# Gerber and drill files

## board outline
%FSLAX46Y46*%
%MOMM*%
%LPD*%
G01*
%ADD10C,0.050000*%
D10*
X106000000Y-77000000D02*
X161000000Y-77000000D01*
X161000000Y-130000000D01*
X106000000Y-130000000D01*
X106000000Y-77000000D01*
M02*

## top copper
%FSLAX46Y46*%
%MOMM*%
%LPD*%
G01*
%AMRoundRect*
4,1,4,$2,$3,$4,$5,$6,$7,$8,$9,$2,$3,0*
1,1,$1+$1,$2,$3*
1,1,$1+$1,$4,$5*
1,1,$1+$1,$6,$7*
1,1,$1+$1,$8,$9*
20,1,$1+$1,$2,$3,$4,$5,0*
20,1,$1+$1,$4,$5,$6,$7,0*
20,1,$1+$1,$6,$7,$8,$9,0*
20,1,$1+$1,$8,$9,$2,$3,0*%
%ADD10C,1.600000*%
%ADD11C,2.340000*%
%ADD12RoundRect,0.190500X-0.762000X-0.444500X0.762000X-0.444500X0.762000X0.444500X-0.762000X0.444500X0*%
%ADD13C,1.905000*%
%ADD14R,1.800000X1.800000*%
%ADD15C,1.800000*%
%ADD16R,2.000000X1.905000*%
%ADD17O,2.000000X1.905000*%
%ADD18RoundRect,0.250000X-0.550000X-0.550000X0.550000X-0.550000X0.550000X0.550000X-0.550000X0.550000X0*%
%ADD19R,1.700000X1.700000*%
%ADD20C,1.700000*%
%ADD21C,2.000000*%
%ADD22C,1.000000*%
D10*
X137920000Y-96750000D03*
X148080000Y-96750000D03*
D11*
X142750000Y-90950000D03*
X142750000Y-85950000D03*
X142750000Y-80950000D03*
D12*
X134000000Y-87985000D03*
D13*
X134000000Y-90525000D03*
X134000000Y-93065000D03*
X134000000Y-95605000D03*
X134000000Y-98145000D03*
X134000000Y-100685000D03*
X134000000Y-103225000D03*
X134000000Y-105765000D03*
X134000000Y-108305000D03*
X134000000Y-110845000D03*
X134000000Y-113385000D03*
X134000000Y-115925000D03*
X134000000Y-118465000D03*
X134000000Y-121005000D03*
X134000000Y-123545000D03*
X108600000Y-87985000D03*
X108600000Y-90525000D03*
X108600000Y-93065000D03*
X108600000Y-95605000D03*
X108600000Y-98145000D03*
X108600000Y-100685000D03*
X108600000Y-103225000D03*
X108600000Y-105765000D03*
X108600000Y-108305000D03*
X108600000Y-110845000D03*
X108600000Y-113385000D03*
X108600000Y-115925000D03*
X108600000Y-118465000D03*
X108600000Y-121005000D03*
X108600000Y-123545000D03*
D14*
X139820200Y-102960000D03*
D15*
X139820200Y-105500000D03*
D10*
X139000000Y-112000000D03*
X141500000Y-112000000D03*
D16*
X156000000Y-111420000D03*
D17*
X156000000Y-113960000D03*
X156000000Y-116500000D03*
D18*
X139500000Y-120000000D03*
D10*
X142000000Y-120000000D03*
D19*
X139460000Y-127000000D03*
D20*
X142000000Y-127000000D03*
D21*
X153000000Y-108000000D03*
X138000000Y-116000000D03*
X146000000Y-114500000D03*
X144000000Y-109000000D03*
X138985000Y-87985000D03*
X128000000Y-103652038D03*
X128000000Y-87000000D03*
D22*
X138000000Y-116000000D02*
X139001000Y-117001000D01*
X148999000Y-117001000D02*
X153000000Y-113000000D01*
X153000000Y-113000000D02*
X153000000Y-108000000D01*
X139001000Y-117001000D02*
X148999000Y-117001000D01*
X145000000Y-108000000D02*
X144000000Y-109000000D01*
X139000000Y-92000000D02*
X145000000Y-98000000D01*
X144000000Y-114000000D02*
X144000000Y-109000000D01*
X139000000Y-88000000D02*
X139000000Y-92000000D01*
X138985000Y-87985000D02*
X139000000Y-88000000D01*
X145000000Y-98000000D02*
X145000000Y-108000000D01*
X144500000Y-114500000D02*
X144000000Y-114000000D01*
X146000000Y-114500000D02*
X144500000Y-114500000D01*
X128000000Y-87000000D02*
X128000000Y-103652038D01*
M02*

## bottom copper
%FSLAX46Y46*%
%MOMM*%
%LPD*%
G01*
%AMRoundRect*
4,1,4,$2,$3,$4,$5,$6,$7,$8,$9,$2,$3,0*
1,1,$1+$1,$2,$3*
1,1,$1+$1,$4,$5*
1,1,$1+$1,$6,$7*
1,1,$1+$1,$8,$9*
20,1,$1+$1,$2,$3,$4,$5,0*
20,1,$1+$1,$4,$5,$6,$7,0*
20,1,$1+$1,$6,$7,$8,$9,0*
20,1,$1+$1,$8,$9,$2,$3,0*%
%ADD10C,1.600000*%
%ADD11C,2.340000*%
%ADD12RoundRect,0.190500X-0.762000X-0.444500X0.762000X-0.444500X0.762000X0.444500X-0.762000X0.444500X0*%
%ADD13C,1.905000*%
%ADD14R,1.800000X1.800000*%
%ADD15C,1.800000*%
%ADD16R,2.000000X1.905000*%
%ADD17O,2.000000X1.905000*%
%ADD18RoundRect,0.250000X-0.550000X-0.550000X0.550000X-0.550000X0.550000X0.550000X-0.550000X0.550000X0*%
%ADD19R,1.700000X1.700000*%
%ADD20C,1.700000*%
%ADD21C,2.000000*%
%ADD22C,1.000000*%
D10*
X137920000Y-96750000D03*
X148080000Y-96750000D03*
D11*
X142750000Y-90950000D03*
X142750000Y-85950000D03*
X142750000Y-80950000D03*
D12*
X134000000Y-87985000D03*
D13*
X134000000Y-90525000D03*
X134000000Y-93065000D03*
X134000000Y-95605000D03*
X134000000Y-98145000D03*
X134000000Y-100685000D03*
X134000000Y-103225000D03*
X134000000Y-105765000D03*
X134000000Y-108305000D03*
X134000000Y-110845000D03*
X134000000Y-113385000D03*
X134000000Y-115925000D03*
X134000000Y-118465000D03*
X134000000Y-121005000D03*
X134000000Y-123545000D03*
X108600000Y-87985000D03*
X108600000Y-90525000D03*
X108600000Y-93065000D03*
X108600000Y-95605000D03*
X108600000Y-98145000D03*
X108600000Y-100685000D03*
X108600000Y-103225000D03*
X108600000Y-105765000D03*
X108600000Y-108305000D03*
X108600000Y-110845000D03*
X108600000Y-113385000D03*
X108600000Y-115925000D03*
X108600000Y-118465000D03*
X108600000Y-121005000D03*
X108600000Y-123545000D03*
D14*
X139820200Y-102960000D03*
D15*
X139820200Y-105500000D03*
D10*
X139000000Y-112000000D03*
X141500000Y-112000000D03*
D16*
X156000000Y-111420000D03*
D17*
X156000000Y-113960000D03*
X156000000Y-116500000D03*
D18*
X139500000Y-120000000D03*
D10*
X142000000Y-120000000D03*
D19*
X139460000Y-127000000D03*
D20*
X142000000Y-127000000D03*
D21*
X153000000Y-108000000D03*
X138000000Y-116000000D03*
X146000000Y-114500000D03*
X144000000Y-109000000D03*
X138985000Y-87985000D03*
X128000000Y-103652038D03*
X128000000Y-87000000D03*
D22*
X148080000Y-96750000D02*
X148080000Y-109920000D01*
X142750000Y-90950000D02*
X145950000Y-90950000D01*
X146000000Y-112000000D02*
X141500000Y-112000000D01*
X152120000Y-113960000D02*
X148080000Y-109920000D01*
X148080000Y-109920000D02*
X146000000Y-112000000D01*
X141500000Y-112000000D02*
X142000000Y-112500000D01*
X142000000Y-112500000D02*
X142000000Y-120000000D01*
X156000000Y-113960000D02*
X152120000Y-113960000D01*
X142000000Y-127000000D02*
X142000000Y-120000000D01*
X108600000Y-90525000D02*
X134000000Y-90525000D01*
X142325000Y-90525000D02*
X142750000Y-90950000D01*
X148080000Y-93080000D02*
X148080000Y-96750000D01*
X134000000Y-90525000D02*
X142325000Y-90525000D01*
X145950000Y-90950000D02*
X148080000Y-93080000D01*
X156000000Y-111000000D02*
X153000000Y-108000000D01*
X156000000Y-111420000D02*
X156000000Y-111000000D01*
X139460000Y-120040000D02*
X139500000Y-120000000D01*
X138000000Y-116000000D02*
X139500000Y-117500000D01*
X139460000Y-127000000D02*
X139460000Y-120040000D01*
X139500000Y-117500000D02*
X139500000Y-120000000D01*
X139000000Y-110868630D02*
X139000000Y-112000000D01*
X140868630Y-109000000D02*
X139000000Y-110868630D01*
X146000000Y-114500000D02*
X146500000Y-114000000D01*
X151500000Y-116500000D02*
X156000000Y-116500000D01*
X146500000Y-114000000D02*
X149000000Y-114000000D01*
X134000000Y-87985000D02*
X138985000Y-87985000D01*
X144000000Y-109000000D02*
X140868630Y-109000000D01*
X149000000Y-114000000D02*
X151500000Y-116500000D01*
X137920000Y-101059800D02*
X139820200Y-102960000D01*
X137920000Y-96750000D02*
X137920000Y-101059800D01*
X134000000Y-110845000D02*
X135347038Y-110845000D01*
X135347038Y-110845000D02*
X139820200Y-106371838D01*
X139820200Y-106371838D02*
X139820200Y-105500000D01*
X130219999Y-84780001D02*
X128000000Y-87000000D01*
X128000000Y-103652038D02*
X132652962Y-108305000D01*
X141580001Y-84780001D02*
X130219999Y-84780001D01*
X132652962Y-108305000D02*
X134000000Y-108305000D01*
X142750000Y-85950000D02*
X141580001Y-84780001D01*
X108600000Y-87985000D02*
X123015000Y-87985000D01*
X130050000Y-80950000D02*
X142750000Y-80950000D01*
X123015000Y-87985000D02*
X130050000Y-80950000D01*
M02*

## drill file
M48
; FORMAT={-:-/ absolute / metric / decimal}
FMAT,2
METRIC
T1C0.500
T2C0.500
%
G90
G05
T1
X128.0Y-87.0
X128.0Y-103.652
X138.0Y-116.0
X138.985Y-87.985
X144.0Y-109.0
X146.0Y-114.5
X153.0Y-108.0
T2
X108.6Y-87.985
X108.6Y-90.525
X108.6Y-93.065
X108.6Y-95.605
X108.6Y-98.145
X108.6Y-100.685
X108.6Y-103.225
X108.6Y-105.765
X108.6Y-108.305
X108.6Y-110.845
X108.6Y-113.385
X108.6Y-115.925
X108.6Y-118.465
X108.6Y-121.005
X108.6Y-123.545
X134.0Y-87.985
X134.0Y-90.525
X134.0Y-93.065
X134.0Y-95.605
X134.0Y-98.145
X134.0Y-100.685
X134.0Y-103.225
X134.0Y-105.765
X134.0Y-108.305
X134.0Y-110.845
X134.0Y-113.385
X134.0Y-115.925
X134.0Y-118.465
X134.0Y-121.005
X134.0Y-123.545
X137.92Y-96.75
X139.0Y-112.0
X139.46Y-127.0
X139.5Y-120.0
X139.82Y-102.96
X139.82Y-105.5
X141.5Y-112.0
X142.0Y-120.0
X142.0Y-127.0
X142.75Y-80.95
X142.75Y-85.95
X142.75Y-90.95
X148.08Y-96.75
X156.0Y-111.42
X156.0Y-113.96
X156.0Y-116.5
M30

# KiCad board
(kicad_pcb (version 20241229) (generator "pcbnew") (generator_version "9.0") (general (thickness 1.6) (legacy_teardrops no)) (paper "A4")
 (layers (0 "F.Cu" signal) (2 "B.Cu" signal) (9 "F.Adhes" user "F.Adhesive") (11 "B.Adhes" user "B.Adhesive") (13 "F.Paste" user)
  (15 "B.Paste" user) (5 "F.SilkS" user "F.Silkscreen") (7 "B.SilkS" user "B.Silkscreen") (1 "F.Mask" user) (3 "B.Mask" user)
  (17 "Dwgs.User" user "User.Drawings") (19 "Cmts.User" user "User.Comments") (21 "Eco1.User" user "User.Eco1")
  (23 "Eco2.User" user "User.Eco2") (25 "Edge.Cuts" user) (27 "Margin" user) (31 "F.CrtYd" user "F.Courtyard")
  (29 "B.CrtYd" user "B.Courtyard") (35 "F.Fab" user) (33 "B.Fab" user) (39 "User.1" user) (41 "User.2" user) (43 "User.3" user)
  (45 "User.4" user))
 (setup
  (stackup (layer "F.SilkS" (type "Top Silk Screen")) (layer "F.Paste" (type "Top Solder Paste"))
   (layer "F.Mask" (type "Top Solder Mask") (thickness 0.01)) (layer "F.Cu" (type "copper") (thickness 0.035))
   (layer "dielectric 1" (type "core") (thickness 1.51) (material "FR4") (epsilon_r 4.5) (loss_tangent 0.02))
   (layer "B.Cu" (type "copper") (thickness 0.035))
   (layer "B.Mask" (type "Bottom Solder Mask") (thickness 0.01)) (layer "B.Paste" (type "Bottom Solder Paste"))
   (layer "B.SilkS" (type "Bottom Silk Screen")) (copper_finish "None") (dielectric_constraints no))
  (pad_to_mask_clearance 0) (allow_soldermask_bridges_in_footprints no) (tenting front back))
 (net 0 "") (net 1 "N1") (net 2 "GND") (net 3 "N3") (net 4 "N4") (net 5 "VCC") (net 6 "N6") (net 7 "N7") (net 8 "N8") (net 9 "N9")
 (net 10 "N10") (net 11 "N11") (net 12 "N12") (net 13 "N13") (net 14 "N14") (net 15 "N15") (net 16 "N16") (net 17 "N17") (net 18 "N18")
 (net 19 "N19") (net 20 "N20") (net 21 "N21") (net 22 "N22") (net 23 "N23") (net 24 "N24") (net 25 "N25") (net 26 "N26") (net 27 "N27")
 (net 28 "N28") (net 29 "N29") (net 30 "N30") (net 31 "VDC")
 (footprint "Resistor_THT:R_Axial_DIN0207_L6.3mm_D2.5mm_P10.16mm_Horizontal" (layer "F.Cu") (at 137.92 96.75)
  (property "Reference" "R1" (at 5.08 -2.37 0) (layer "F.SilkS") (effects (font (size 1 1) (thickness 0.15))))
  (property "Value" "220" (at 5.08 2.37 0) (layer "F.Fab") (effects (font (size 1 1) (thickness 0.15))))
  (pad "1" thru_hole circle (at 0 0) (size 1.6 1.6) (drill 0.5) (layers "*.Cu" "*.Mask") (remove_unused_layers no) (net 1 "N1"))
  (pad "2" thru_hole circle (at 10.16 0) (size 1.6 1.6) (drill 0.5) (layers "*.Cu" "*.Mask") (remove_unused_layers no) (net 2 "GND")))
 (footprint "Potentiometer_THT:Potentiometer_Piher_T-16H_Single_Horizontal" (layer "F.Cu") (at 142.75 90.95)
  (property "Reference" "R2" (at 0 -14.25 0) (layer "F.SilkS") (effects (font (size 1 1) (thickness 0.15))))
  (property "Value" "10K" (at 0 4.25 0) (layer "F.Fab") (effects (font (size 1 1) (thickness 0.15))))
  (pad "1" thru_hole circle (at 0 0) (size 2.34 2.34) (drill 0.5) (layers "*.Cu" "*.Mask") (remove_unused_layers no) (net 2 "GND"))
  (pad "2" thru_hole circle (at 0 -5) (size 2.34 2.34) (drill 0.5) (layers "*.Cu" "*.Mask") (remove_unused_layers no) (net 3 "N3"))
  (pad "3" thru_hole circle (at 0 -10) (size 2.34 2.34) (drill 0.5) (layers "*.Cu" "*.Mask") (remove_unused_layers no) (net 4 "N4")))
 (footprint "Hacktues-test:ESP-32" (layer "F.Cu") (at 121.3 103.225)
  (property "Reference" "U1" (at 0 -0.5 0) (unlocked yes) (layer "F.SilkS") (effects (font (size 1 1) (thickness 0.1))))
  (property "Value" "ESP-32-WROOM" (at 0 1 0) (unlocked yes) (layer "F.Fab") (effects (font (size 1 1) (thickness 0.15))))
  (pad "1" thru_hole roundrect (at 12.7 -15.24) (size 1.905 1.27) (drill 0.5) (layers "*.Cu" "*.Mask") (remove_unused_layers no)
   (roundrect_rratio 0.15) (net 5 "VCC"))
  (pad "2" thru_hole circle (at 12.7 -12.7) (size 1.905 1.905) (drill 0.5) (layers "*.Cu" "*.Mask") (remove_unused_layers no) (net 2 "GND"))
  (pad "3" thru_hole circle (at 12.7 -10.16) (size 1.905 1.905) (drill 0.5) (layers "*.Cu" "*.Mask") (remove_unused_layers no) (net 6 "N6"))
  (pad "4" thru_hole circle (at 12.7 -7.62) (size 1.905 1.905) (drill 0.5) (layers "*.Cu" "*.Mask") (remove_unused_layers no) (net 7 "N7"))
  (pad "5" thru_hole circle (at 12.7 -5.08) (size 1.905 1.905) (drill 0.5) (layers "*.Cu" "*.Mask") (remove_unused_layers no) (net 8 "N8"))
  (pad "6" thru_hole circle (at 12.7 -2.54) (size 1.905 1.905) (drill 0.5) (layers "*.Cu" "*.Mask") (remove_unused_layers no) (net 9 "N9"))
  (pad "7" thru_hole circle (at 12.7 0) (size 1.905 1.905) (drill 0.5) (layers "*.Cu" "*.Mask") (remove_unused_layers no) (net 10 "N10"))
  (pad "8" thru_hole circle (at 12.7 2.54) (size 1.905 1.905) (drill 0.5) (layers "*.Cu" "*.Mask") (remove_unused_layers no) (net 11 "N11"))
  (pad "9" thru_hole circle (at 12.7 5.08) (size 1.905 1.905) (drill 0.5) (layers "*.Cu" "*.Mask") (remove_unused_layers no) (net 3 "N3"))
  (pad "10" thru_hole circle (at 12.7 7.62) (size 1.905 1.905) (drill 0.5) (layers "*.Cu" "*.Mask") (remove_unused_layers no) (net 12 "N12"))
  (pad "11" thru_hole circle (at 12.7 10.16) (size 1.905 1.905) (drill 0.5) (layers "*.Cu" "*.Mask") (remove_unused_layers no)
   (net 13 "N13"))
  (pad "12" thru_hole circle (at 12.7 12.7) (size 1.905 1.905) (drill 0.5) (layers "*.Cu" "*.Mask") (remove_unused_layers no) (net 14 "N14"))
  (pad "13" thru_hole circle (at 12.7 15.24) (size 1.905 1.905) (drill 0.5) (layers "*.Cu" "*.Mask") (remove_unused_layers no)
   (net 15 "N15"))
  (pad "14" thru_hole circle (at 12.7 17.78) (size 1.905 1.905) (drill 0.5) (layers "*.Cu" "*.Mask") (remove_unused_layers no)
   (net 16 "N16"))
  (pad "15" thru_hole circle (at 12.7 20.32) (size 1.905 1.905) (drill 0.5) (layers "*.Cu" "*.Mask") (remove_unused_layers no)
   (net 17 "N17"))
  (pad "16" thru_hole circle (at -12.7 -15.24) (size 1.905 1.905) (drill 0.5) (layers "*.Cu" "*.Mask") (remove_unused_layers no)
   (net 4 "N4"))
  (pad "17" thru_hole circle (at -12.7 -12.7) (size 1.905 1.905) (drill 0.5) (layers "*.Cu" "*.Mask") (remove_unused_layers no)
   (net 2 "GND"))
  (pad "18" thru_hole circle (at -12.7 -10.16) (size 1.905 1.905) (drill 0.5) (layers "*.Cu" "*.Mask") (remove_unused_layers no)
   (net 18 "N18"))
  (pad "19" thru_hole circle (at -12.7 -7.62) (size 1.905 1.905) (drill 0.5) (layers "*.Cu" "*.Mask") (remove_unused_layers no)
   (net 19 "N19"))
  (pad "20" thru_hole circle (at -12.7 -5.08) (size 1.905 1.905) (drill 0.5) (layers "*.Cu" "*.Mask") (remove_unused_layers no)
   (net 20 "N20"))
  (pad "21" thru_hole circle (at -12.7 -2.54) (size 1.905 1.905) (drill 0.5) (layers "*.Cu" "*.Mask") (remove_unused_layers no)
   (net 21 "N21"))
  (pad "22" thru_hole circle (at -12.7 0) (size 1.905 1.905) (drill 0.5) (layers "*.Cu" "*.Mask") (remove_unused_layers no) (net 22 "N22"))
  (pad "23" thru_hole circle (at -12.7 2.54) (size 1.905 1.905) (drill 0.5) (layers "*.Cu" "*.Mask") (remove_unused_layers no)
   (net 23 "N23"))
  (pad "24" thru_hole circle (at -12.7 5.08) (size 1.905 1.905) (drill 0.5) (layers "*.Cu" "*.Mask") (remove_unused_layers no)
   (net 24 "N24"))
  (pad "25" thru_hole circle (at -12.7 7.62) (size 1.905 1.905) (drill 0.5) (layers "*.Cu" "*.Mask") (remove_unused_layers no)
   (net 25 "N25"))
  (pad "26" thru_hole circle (at -12.7 10.16) (size 1.905 1.905) (drill 0.5) (layers "*.Cu" "*.Mask") (remove_unused_layers no)
   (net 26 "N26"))
  (pad "27" thru_hole circle (at -12.7 12.7) (size 1.905 1.905) (drill 0.5) (layers "*.Cu" "*.Mask") (remove_unused_layers no)
   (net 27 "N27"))
  (pad "28" thru_hole circle (at -12.7 15.24) (size 1.905 1.905) (drill 0.5) (layers "*.Cu" "*.Mask") (remove_unused_layers no)
   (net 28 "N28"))
  (pad "29" thru_hole circle (at -12.7 17.78) (size 1.905 1.905) (drill 0.5) (layers "*.Cu" "*.Mask") (remove_unused_layers no)
   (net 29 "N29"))
  (pad "30" thru_hole circle (at -12.7 20.32) (size 1.905 1.905) (drill 0.5) (layers "*.Cu" "*.Mask") (remove_unused_layers no)
   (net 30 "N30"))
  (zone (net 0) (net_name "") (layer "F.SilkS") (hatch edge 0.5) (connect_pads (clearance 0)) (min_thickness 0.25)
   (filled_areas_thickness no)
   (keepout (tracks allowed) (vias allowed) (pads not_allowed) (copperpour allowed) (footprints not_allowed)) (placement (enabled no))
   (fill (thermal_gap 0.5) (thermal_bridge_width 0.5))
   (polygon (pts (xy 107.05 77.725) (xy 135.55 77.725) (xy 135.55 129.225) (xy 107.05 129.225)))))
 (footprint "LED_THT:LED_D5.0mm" (layer "F.Cu") (at 139.8202 102.96 -90)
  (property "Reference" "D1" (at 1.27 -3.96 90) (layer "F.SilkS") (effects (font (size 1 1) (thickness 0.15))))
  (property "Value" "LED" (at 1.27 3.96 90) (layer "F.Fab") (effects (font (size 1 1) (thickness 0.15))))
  (pad "1" thru_hole rect (at 0 0 270) (size 1.8 1.8) (drill 0.5) (layers "*.Cu" "*.Mask") (remove_unused_layers no) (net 1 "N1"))
  (pad "2" thru_hole circle (at 2.54 0 270) (size 1.8 1.8) (drill 0.5) (layers "*.Cu" "*.Mask") (remove_unused_layers no) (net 12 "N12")))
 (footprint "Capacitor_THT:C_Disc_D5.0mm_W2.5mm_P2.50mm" (layer "F.Cu") (at 139 112)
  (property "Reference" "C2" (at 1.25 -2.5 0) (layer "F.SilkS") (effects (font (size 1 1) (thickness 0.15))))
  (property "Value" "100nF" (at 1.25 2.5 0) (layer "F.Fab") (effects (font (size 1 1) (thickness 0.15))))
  (pad "1" thru_hole circle (at 0 0) (size 1.6 1.6) (drill 0.5) (layers "*.Cu" "*.Mask") (remove_unused_layers no) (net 5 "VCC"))
  (pad "2" thru_hole circle (at 2.5 0) (size 1.6 1.6) (drill 0.5) (layers "*.Cu" "*.Mask") (remove_unused_layers no) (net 2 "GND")))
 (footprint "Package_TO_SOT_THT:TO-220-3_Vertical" (layer "F.Cu") (at 156 111.42 -90)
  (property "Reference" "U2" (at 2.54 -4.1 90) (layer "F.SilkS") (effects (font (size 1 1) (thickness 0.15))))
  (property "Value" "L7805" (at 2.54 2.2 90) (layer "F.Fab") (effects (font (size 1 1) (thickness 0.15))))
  (pad "1" thru_hole rect (at 0 0 270) (size 1.905 2) (drill 0.5) (layers "*.Cu" "*.Mask") (remove_unused_layers no) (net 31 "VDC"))
  (pad "2" thru_hole oval (at 2.54 0 270) (size 1.905 2) (drill 0.5) (layers "*.Cu" "*.Mask") (remove_unused_layers no) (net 2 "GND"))
  (pad "3" thru_hole oval (at 5.08 0 270) (size 1.905 2) (drill 0.5) (layers "*.Cu" "*.Mask") (remove_unused_layers no) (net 5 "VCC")))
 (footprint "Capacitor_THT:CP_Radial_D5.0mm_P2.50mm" (layer "F.Cu") (at 139.5 120)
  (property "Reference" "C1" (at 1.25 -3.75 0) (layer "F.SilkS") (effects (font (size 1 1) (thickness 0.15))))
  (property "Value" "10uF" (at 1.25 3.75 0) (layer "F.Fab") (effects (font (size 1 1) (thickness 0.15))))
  (pad "1" thru_hole roundrect (at 0 0) (size 1.6 1.6) (drill 0.5) (layers "*.Cu" "*.Mask") (remove_unused_layers no)
   (roundrect_rratio 0.15625) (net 31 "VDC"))
  (pad "2" thru_hole circle (at 2.5 0) (size 1.6 1.6) (drill 0.5) (layers "*.Cu" "*.Mask") (remove_unused_layers no) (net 2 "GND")))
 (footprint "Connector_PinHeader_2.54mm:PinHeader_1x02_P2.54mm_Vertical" (layer "F.Cu") (at 139.46 127 90)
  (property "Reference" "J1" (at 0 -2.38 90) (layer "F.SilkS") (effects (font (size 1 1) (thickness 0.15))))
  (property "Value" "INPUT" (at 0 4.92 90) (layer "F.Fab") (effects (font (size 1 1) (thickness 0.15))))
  (pad "1" thru_hole rect (at 0 0 90) (size 1.7 1.7) (drill 0.5) (layers "*.Cu" "*.Mask") (remove_unused_layers no) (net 31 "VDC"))
  (pad "2" thru_hole circle (at 0 2.54 90) (size 1.7 1.7) (drill 0.5) (layers "*.Cu" "*.Mask") (remove_unused_layers no) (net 2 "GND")))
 (gr_rect (start 106 77) (end 161 130) (stroke (width 0.05) (type default)) (fill no) (layer "Edge.Cuts"))
 (segment (start 148.08 96.75) (end 148.08 109.92) (width 1) (layer "B.Cu") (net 2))
 (segment (start 142.75 90.95) (end 145.95 90.95) (width 1) (layer "B.Cu") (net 2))
 (segment (start 146 112) (end 141.5 112) (width 1) (layer "B.Cu") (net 2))
 (segment (start 152.12 113.96) (end 148.08 109.92) (width 1) (layer "B.Cu") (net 2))
 (segment (start 148.08 109.92) (end 146 112) (width 1) (layer "B.Cu") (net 2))
 (segment (start 141.5 112) (end 142 112.5) (width 1) (layer "B.Cu") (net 2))
 (segment (start 142 112.5) (end 142 120) (width 1) (layer "B.Cu") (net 2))
 (segment (start 156 113.96) (end 152.12 113.96) (width 1) (layer "B.Cu") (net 2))
 (segment (start 142 127) (end 142 120) (width 1) (layer "B.Cu") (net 2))
 (segment (start 108.6 90.525) (end 134 90.525) (width 1) (layer "B.Cu") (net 2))
 (segment (start 142.325 90.525) (end 142.75 90.95) (width 1) (layer "B.Cu") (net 2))
 (segment (start 148.08 93.08) (end 148.08 96.75) (width 1) (layer "B.Cu") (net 2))
 (segment (start 134 90.525) (end 142.325 90.525) (width 1) (layer "B.Cu") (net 2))
 (segment (start 145.95 90.95) (end 148.08 93.08) (width 1) (layer "B.Cu") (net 2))
 (segment (start 138 116) (end 139.001 117.001) (width 1) (layer "F.Cu") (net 31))
 (segment (start 148.999 117.001) (end 153 113) (width 1) (layer "F.Cu") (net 31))
 (segment (start 153 113) (end 153 108) (width 1) (layer "F.Cu") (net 31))
 (segment (start 139.001 117.001) (end 148.999 117.001) (width 1) (layer "F.Cu") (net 31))
 (via (at 153 108) (size 2) (drill 0.5) (layers "F.Cu" "B.Cu") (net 31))
 (via (at 138 116) (size 2) (drill 0.5) (layers "F.Cu" "B.Cu") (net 31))
 (segment (start 156 111) (end 153 108) (width 1) (layer "B.Cu") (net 31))
 (segment (start 156 111.42) (end 156 111) (width 1) (layer "B.Cu") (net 31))
 (segment (start 139.46 120.04) (end 139.5 120) (width 1) (layer "B.Cu") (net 31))
 (segment (start 138 116) (end 139.5 117.5) (width 1) (layer "B.Cu") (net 31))
 (segment (start 139.46 127) (end 139.46 120.04) (width 1) (layer "B.Cu") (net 31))
 (segment (start 139.5 117.5) (end 139.5 120) (width 1) (layer "B.Cu") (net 31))
 (segment (start 145 108) (end 144 109) (width 1) (layer "F.Cu") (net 5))
 (segment (start 139 92) (end 145 98) (width 1) (layer "F.Cu") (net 5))
 (segment (start 144 114) (end 144 109) (width 1) (layer "F.Cu") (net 5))
 (segment (start 139 88) (end 139 92) (width 1) (layer "F.Cu") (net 5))
 (segment (start 138.985 87.985) (end 139 88) (width 1) (layer "F.Cu") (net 5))
 (segment (start 145 98) (end 145 108) (width 1) (layer "F.Cu") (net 5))
 (segment (start 144.5 114.5) (end 144 114) (width 1) (layer "F.Cu") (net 5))
 (segment (start 146 114.5) (end 144.5 114.5) (width 1) (layer "F.Cu") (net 5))
 (via (at 146 114.5) (size 2) (drill 0.5) (layers "F.Cu" "B.Cu") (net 5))
 (via (at 144 109) (size 2) (drill 0.5) (layers "F.Cu" "B.Cu") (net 5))
 (via (at 138.985 87.985) (size 2) (drill 0.5) (layers "F.Cu" "B.Cu") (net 5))
 (segment (start 139 110.86863) (end 139 112) (width 1) (layer "B.Cu") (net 5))
 (segment (start 140.86863 109) (end 139 110.86863) (width 1) (layer "B.Cu") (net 5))
 (segment (start 146 114.5) (end 146.5 114) (width 1) (layer "B.Cu") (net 5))
 (segment (start 151.5 116.5) (end 156 116.5) (width 1) (layer "B.Cu") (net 5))
 (segment (start 146.5 114) (end 149 114) (width 1) (layer "B.Cu") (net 5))
 (segment (start 134 87.985) (end 138.985 87.985) (width 1) (layer "B.Cu") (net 5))
 (segment (start 144 109) (end 140.86863 109) (width 1) (layer "B.Cu") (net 5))
 (segment (start 149 114) (end 151.5 116.5) (width 1) (layer "B.Cu") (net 5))
 (segment (start 137.92 101.0598) (end 139.8202 102.96) (width 1) (layer "B.Cu") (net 1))
 (segment (start 137.92 96.75) (end 137.92 101.0598) (width 1) (layer "B.Cu") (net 1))
 (segment (start 134 110.845) (end 135.347038 110.845) (width 1) (layer "B.Cu") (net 12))
 (segment (start 135.347038 110.845) (end 139.8202 106.371838) (width 1) (layer "B.Cu") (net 12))
 (segment (start 139.8202 106.371838) (end 139.8202 105.5) (width 1) (layer "B.Cu") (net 12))
 (segment (start 128 87) (end 128 103.652038) (width 1) (layer "F.Cu") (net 3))
 (via (at 128 103.652038) (size 2) (drill 0.5) (layers "F.Cu" "B.Cu") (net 3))
 (via (at 128 87) (size 2) (drill 0.5) (layers "F.Cu" "B.Cu") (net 3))
 (segment (start 130.219999 84.780001) (end 128 87) (width 1) (layer "B.Cu") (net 3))
 (segment (start 128 103.652038) (end 132.652962 108.305) (width 1) (layer "B.Cu") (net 3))
 (segment (start 141.580001 84.780001) (end 130.219999 84.780001) (width 1) (layer "B.Cu") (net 3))
 (segment (start 132.652962 108.305) (end 134 108.305) (width 1) (layer "B.Cu") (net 3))
 (segment (start 142.75 85.95) (end 141.580001 84.780001) (width 1) (layer "B.Cu") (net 3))
 (segment (start 108.6 87.985) (end 123.015 87.985) (width 1) (layer "B.Cu") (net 4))
 (segment (start 130.05 80.95) (end 142.75 80.95) (width 1) (layer "B.Cu") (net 4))
 (segment (start 123.015 87.985) (end 130.05 80.95) (width 1) (layer "B.Cu") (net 4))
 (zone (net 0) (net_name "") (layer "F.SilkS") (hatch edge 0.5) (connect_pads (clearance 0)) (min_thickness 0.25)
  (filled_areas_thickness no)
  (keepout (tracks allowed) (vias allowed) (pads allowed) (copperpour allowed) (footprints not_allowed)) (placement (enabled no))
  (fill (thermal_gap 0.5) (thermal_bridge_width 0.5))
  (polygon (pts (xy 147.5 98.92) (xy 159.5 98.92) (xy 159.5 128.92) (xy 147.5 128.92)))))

